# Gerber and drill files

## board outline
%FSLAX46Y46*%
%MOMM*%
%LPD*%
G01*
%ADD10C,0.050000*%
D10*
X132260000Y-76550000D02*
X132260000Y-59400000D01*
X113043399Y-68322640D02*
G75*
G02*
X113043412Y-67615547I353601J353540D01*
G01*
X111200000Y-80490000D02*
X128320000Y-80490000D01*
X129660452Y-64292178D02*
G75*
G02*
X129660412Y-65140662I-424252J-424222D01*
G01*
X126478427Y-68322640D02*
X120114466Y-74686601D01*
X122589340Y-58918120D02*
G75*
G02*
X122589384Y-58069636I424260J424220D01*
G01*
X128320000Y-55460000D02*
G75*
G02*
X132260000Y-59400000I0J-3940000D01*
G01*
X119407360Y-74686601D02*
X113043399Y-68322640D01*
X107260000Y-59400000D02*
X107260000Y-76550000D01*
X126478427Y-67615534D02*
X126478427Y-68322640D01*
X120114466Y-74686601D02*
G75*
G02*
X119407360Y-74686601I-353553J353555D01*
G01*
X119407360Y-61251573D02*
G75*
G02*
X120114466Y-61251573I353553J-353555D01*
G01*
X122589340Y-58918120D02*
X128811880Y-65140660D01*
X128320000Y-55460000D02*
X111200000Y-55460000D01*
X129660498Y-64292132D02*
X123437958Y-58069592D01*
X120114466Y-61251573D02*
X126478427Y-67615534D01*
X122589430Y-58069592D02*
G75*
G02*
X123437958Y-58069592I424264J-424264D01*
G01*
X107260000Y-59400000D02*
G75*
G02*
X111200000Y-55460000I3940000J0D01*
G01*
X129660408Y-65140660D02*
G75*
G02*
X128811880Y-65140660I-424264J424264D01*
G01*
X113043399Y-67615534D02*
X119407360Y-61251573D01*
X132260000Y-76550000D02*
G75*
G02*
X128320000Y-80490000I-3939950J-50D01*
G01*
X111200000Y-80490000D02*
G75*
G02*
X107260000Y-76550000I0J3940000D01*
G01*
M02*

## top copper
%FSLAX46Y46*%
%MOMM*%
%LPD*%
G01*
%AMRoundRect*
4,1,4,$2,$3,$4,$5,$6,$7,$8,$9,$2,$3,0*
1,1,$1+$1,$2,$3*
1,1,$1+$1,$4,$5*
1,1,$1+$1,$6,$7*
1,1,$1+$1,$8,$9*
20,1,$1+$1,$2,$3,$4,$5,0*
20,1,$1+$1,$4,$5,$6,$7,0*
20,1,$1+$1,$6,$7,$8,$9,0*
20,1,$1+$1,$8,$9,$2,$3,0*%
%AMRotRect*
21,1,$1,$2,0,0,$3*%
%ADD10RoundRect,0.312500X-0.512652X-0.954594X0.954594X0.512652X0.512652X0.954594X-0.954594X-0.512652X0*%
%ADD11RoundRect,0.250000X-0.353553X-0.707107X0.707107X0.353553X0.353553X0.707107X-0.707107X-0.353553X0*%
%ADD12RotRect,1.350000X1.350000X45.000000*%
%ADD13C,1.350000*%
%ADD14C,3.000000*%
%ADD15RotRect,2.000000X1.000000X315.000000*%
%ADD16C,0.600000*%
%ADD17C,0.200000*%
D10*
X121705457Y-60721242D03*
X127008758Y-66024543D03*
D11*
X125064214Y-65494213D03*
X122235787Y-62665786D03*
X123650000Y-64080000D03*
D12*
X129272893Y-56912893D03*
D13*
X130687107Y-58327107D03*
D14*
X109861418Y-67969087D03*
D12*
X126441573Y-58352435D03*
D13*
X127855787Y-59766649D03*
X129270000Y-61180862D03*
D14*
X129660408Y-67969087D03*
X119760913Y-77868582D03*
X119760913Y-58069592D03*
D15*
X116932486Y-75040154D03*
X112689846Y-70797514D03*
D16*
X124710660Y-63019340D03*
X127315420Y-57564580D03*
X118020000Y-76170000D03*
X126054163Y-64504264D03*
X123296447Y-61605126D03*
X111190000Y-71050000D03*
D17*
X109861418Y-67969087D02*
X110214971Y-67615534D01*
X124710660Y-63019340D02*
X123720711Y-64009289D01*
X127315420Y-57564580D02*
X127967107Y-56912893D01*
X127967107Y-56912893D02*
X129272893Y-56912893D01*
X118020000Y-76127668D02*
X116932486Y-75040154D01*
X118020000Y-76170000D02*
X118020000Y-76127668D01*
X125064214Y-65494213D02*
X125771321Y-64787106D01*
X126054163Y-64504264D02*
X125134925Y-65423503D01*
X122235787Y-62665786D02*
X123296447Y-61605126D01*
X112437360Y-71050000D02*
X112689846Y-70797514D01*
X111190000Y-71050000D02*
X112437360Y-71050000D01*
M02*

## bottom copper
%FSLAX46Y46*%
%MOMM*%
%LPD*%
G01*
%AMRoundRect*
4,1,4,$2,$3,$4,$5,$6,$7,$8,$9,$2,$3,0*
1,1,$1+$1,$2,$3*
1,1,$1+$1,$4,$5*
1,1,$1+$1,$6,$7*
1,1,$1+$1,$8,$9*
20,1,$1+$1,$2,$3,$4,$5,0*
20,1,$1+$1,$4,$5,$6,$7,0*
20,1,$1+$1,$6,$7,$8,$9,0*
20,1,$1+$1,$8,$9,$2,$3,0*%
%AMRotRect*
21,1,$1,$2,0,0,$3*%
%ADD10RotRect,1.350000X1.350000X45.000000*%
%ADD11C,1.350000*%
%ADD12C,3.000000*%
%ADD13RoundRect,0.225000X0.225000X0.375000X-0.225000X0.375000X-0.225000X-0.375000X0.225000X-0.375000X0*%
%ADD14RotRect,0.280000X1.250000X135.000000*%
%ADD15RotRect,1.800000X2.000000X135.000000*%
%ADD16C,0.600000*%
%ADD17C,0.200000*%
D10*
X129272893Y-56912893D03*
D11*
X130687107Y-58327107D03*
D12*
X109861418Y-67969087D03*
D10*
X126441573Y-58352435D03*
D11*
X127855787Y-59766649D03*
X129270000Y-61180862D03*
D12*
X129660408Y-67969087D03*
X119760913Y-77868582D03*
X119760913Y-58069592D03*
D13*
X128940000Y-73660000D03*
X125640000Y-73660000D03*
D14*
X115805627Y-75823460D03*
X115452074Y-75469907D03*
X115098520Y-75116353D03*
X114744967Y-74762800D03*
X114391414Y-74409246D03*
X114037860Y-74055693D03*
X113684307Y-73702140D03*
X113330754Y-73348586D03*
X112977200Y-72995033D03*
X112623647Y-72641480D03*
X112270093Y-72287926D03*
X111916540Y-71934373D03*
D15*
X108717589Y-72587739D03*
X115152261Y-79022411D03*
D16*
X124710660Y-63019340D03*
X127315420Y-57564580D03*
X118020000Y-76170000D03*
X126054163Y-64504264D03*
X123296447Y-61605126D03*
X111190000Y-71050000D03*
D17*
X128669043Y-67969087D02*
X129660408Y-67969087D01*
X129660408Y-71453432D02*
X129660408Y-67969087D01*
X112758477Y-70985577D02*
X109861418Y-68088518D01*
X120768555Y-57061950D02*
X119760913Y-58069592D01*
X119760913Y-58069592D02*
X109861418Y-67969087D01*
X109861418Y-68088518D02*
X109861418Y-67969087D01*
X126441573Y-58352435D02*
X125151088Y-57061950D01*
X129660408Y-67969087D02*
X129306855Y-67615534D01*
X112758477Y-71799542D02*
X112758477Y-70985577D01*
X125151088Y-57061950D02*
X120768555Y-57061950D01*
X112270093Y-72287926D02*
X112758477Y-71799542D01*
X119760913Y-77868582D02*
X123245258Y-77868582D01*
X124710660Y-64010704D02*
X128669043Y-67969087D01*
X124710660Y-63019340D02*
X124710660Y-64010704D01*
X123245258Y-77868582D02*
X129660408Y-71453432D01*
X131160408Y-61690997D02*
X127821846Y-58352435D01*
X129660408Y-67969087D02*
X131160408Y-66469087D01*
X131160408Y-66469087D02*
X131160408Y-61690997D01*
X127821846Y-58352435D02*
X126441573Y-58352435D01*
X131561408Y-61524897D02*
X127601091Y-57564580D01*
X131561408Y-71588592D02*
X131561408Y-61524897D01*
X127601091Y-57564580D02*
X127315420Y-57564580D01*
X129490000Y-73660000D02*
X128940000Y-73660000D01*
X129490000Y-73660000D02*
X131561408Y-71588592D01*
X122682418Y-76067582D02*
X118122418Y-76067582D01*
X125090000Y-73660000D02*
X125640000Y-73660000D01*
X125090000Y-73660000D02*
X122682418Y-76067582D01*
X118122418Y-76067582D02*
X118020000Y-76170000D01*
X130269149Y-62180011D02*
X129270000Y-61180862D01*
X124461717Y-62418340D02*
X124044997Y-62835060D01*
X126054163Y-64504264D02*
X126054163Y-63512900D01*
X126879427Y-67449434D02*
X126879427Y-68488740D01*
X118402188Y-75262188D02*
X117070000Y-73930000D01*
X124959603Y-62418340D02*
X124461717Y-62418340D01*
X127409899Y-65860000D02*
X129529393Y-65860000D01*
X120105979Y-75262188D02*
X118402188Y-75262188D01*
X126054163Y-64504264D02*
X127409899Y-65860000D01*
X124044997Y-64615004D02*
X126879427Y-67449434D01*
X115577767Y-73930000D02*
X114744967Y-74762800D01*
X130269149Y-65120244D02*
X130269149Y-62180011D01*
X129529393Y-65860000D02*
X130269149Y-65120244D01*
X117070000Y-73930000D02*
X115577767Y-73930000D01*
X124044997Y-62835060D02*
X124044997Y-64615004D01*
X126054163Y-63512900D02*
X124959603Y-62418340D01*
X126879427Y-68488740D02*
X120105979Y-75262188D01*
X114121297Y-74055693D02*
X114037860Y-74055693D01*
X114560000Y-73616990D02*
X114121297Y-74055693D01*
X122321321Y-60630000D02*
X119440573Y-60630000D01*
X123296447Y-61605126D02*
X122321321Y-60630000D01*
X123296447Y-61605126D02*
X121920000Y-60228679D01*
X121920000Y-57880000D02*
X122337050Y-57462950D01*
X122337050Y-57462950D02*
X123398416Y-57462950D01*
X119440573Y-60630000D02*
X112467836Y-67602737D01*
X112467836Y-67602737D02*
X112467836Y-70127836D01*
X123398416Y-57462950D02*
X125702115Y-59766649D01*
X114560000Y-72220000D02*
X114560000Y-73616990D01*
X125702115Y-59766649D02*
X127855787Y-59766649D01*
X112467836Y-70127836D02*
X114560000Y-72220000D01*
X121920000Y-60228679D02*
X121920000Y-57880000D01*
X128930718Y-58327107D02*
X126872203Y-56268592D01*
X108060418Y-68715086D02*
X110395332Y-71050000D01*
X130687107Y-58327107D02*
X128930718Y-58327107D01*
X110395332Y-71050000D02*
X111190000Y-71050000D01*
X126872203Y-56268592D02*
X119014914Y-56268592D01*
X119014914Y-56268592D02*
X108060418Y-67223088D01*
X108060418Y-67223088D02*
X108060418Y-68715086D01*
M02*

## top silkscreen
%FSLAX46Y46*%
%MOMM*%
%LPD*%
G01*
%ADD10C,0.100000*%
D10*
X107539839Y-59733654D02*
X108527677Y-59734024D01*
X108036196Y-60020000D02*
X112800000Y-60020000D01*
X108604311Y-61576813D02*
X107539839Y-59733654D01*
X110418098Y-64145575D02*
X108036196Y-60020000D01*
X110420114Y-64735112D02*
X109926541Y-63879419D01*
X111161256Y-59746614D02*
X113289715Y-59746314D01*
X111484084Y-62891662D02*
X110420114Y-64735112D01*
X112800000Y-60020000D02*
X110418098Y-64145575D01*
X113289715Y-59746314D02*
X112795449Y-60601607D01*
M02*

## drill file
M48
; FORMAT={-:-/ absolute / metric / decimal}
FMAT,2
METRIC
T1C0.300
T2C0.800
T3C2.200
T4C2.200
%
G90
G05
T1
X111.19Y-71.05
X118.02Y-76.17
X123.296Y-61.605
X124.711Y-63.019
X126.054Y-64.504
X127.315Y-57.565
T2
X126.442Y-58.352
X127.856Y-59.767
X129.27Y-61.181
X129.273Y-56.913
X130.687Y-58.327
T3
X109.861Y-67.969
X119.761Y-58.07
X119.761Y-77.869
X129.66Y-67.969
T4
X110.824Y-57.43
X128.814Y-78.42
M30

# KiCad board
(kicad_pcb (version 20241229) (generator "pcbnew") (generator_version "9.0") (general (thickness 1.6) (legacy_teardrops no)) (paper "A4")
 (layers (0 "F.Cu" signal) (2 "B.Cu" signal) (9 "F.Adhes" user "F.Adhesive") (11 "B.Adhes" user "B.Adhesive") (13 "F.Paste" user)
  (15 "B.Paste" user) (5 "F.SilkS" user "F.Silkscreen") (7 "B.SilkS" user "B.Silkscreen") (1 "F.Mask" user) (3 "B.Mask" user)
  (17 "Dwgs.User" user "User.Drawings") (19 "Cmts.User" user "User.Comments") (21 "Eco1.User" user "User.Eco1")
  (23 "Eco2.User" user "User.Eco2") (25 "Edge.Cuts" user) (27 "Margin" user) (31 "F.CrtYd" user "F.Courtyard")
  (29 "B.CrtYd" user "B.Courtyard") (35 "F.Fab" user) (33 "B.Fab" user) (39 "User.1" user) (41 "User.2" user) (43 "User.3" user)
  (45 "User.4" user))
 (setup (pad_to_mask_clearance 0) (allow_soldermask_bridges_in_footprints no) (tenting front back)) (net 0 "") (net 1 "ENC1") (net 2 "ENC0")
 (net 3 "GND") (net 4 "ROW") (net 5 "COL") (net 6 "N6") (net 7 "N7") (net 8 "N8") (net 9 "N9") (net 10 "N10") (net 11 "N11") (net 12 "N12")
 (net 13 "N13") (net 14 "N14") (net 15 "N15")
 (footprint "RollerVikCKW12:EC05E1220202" (layer "F.Cu") (at 119.760913 67.969087 45)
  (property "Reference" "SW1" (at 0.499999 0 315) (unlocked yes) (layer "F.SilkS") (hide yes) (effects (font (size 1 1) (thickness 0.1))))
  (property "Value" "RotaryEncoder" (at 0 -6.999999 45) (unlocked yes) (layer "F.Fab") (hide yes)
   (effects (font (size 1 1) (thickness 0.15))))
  (pad "" smd roundrect (at 6.500001 -3.75 45) (size 2.7 1.25) (layers "F.Cu" "F.Mask" "F.Paste") (roundrect_rratio 0.25)
   (thermal_bridge_angle 45))
  (pad "" smd roundrect (at 6.500001 3.75 45) (size 2.7 1.25) (layers "F.Cu" "F.Mask" "F.Paste") (roundrect_rratio 0.25)
   (thermal_bridge_angle 45))
  (pad "A" smd roundrect (at 5.5 2 45) (size 2 1) (layers "F.Cu" "F.Mask" "F.Paste") (roundrect_rratio 0.25) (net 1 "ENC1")
   (thermal_bridge_angle 45))
  (pad "B" smd roundrect (at 5.5 -2 45) (size 2 1) (layers "F.Cu" "F.Mask" "F.Paste") (roundrect_rratio 0.25) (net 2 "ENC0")
   (thermal_bridge_angle 45))
  (pad "C" smd roundrect (at 5.5 0 45) (size 2 1) (layers "F.Cu" "F.Mask" "F.Paste") (roundrect_rratio 0.25) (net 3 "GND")
   (thermal_bridge_angle 45)))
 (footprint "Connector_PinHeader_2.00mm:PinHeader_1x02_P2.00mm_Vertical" (layer "F.Cu") (at 129.272893 56.912893 45)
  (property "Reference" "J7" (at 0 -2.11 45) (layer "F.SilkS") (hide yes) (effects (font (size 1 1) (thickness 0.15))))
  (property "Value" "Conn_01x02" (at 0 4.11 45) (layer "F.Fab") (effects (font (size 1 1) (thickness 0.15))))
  (pad "1" thru_hole rect (at 0 0 45) (size 1.35 1.35) (drill 0.8) (layers "*.Cu" "*.Mask") (remove_unused_layers no) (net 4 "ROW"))
  (pad "2" thru_hole circle (at 0 2.000001 45) (size 1.35 1.35) (drill 0.8) (layers "*.Cu" "*.Mask") (remove_unused_layers no) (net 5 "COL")))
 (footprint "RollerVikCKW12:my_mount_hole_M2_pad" (layer "F.Cu") (at 109.861418 67.969087 -45)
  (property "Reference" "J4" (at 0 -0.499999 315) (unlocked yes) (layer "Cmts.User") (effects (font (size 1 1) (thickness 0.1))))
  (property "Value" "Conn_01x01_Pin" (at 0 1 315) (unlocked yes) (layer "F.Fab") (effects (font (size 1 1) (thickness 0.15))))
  (pad "1" thru_hole circle (at 0 0 315) (size 3 3) (drill 2.2) (layers "*.Cu" "*.Mask") (remove_unused_layers no) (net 3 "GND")))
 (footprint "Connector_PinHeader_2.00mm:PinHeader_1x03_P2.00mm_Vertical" (layer "F.Cu") (at 126.441573 58.352435 45)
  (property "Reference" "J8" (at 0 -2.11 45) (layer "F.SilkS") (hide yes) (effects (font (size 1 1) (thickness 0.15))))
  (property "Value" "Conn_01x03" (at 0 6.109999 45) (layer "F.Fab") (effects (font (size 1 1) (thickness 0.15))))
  (pad "1" thru_hole rect (at 0 0 45) (size 1.35 1.35) (drill 0.8) (layers "*.Cu" "*.Mask") (remove_unused_layers no) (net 3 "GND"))
  (pad "2" thru_hole circle (at 0 2.000001 45) (size 1.35 1.35) (drill 0.8) (layers "*.Cu" "*.Mask") (remove_unused_layers no)
   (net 2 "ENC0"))
  (pad "3" thru_hole circle (at 0 4 45) (size 1.35 1.35) (drill 0.8) (layers "*.Cu" "*.Mask") (remove_unused_layers no) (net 1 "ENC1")))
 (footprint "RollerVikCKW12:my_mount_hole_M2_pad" (layer "F.Cu") (at 129.660408 67.969087 45)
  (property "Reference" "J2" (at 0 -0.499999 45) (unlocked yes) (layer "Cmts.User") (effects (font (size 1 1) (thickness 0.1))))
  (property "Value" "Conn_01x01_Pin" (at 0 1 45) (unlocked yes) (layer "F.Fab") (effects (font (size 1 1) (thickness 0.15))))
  (pad "1" thru_hole circle (at 0 0 45) (size 3 3) (drill 2.2) (layers "*.Cu" "*.Mask") (remove_unused_layers no) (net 3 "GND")))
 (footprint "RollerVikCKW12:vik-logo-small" (layer "F.Cu") (at 110.42 61.54)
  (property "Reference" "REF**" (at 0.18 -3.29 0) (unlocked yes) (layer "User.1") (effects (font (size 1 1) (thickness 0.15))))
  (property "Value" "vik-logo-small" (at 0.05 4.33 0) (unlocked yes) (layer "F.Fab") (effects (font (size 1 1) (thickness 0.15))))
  (fp_line (start -2.880161 -1.806346) (end -1.892323 -1.805976) (stroke (width 0.1) (type solid)) (layer "F.SilkS"))
  (fp_line (start -2.383804 -1.52) (end 2.38 -1.52) (stroke (width 0.1) (type solid)) (layer "F.SilkS"))
  (fp_line (start -1.815689 0.036813) (end -2.880161 -1.806346) (stroke (width 0.1) (type solid)) (layer "F.SilkS"))
  (fp_line (start -0.001902 2.605575) (end -2.383804 -1.52) (stroke (width 0.1) (type solid)) (layer "F.SilkS"))
  (fp_line (start 0.000114 3.195112) (end -0.493459 2.339419) (stroke (width 0.1) (type solid)) (layer "F.SilkS"))
  (fp_line (start 0.741256 -1.793386) (end 2.869715 -1.793686) (stroke (width 0.1) (type solid)) (layer "F.SilkS"))
  (fp_line (start 1.064084 1.351662) (end 0.000114 3.195112) (stroke (width 0.1) (type solid)) (layer "F.SilkS"))
  (fp_line (start 2.38 -1.52) (end -0.001902 2.605575) (stroke (width 0.1) (type solid)) (layer "F.SilkS"))
  (fp_line (start 2.869715 -1.793686) (end 2.375449 -0.938393) (stroke (width 0.1) (type solid)) (layer "F.SilkS")))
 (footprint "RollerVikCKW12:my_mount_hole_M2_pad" (layer "F.Cu") (at 119.760913 77.868582 135)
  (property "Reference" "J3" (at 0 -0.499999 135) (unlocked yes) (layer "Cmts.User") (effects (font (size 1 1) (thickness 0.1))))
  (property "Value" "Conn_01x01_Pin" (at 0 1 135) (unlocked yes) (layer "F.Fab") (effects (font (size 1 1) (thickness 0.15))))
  (pad "1" thru_hole circle (at 0 0 135) (size 3 3) (drill 2.2) (layers "*.Cu" "*.Mask") (remove_unused_layers no) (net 3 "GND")))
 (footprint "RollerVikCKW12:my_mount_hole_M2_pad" (layer "F.Cu") (at 119.760913 58.069592 45)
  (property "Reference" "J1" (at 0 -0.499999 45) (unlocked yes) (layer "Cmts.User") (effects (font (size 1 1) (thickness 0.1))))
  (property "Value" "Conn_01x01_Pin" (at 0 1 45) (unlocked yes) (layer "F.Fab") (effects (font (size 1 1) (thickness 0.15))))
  (pad "1" thru_hole circle (at 0 0 45) (size 3 3) (drill 2.2) (layers "*.Cu" "*.Mask") (remove_unused_layers no) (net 3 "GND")))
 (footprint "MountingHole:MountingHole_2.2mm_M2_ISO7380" (layer "F.Cu") (at 110.823806 57.429728)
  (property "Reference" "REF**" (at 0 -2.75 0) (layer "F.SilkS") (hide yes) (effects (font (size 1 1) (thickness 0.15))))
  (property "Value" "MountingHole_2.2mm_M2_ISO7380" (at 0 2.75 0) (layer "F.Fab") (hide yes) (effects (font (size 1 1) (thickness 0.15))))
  (pad "" np_thru_hole circle (at 0 0) (size 2.2 2.2) (drill 2.2) (layers "*.Cu" "*.Mask")))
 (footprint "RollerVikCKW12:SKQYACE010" (layer "F.Cu") (at 114.811166 72.918834 -45)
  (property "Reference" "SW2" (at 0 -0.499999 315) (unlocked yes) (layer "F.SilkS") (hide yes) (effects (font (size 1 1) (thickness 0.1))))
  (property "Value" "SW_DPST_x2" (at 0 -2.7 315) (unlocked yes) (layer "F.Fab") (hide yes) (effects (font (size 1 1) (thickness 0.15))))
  (pad "1" smd rect (at 3 0 315) (size 2 1) (layers "F.Cu" "F.Mask" "F.Paste") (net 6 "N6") (thermal_bridge_angle 45))
  (pad "2" smd rect (at -3 0 315) (size 2 1) (layers "F.Cu" "F.Mask" "F.Paste") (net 5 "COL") (thermal_bridge_angle 45)))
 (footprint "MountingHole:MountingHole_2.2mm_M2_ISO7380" (layer "F.Cu") (at 128.813806 78.419728 90)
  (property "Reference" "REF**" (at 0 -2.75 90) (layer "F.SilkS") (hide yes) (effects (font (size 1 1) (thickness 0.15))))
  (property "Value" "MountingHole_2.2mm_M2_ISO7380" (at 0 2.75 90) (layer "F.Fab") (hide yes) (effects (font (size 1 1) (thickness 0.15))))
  (pad "" np_thru_hole circle (at 0 0 90) (size 2.2 2.2) (drill 2.2) (layers "*.Cu" "*.Mask")))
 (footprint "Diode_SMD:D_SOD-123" (layer "B.Cu") (at 127.29 73.66 180)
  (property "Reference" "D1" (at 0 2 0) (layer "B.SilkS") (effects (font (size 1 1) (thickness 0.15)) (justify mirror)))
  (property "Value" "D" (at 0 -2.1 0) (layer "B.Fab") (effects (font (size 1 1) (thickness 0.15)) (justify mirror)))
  (pad "1" smd roundrect (at -1.65 0 180) (size 0.9 1.2) (layers "B.Cu" "B.Mask" "B.Paste") (roundrect_rratio 0.25) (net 4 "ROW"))
  (pad "2" smd roundrect (at 1.65 0 180) (size 0.9 1.2) (layers "B.Cu" "B.Mask" "B.Paste") (roundrect_rratio 0.25) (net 6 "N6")))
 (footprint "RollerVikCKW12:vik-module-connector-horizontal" (layer "B.Cu") (at 112.42 75.32 135)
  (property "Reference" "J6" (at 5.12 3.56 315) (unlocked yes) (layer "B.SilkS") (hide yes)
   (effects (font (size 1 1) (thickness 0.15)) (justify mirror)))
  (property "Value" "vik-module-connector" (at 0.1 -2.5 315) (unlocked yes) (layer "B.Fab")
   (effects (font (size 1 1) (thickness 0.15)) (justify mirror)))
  (pad "1" smd rect (at -2.75 2.038 135) (size 0.28 1.25) (layers "B.Cu" "B.Mask" "B.Paste") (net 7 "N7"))
  (pad "2" smd rect (at -2.25 2.038 135) (size 0.28 1.25) (layers "B.Cu" "B.Mask" "B.Paste") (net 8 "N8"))
  (pad "3" smd rect (at -1.749999 2.038 135) (size 0.28 1.25) (layers "B.Cu" "B.Mask" "B.Paste") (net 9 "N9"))
  (pad "4" smd rect (at -1.25 2.038 135) (size 0.28 1.25) (layers "B.Cu" "B.Mask" "B.Paste") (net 1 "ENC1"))
  (pad "5" smd rect (at -0.75 2.038001 135) (size 0.28 1.25) (layers "B.Cu" "B.Mask" "B.Paste") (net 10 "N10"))
  (pad "6" smd rect (at -0.25 2.038 135) (size 0.28 1.25) (layers "B.Cu" "B.Mask" "B.Paste") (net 2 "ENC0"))
  (pad "7" smd rect (at 0.25 2.038 135) (size 0.28 1.25) (layers "B.Cu" "B.Mask" "B.Paste") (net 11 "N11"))
  (pad "8" smd rect (at 0.75 2.038001 135) (size 0.28 1.25) (layers "B.Cu" "B.Mask" "B.Paste") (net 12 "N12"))
  (pad "9" smd rect (at 1.25 2.038 135) (size 0.28 1.25) (layers "B.Cu" "B.Mask" "B.Paste") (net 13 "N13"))
  (pad "10" smd rect (at 1.749999 2.038 135) (size 0.28 1.25) (layers "B.Cu" "B.Mask" "B.Paste") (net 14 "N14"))
  (pad "11" smd rect (at 2.25 2.038 135) (size 0.28 1.25) (layers "B.Cu" "B.Mask" "B.Paste") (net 3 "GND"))
  (pad "12" smd rect (at 2.75 2.038 135) (size 0.28 1.25) (layers "B.Cu" "B.Mask" "B.Paste") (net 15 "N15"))
  (pad "13" smd rect (at 4.55 -0.686 135) (size 1.8 2) (layers "B.Cu" "B.Mask" "B.Paste"))
  (pad "14" smd rect (at -4.55 -0.686 135) (size 1.8 2) (layers "B.Cu" "B.Mask" "B.Paste")))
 (gr_line (start 132.26 76.55) (end 132.26 59.4) (stroke (width 0.05) (type solid)) (layer "Edge.Cuts"))
 (gr_arc (start 113.043399 68.32264) (mid 112.896953 67.969087) (end 113.043399 67.615534) (stroke (width 0.05) (type default))
  (layer "Edge.Cuts"))
 (gr_line (start 111.2 80.49) (end 128.32 80.49) (stroke (width 0.05) (type solid)) (layer "Edge.Cuts"))
 (gr_arc (start 129.660452 64.292178) (mid 129.836169 64.716427) (end 129.660408 65.140658) (stroke (width 0.05) (type default))
  (layer "Edge.Cuts"))
 (gr_line (start 126.478427 68.32264) (end 120.114466 74.686601) (stroke (width 0.05) (type default)) (layer "Edge.Cuts"))
 (gr_arc (start 122.58934 58.91812) (mid 122.413604 58.493856) (end 122.58934 58.069592) (stroke (width 0.05) (type default))
  (layer "Edge.Cuts"))
 (gr_arc (start 128.32 55.46) (mid 131.10601 56.61399) (end 132.26 59.4) (stroke (width 0.05) (type solid)) (layer "Edge.Cuts"))
 (gr_line (start 119.40736 74.686601) (end 113.043399 68.32264) (stroke (width 0.05) (type default)) (layer "Edge.Cuts"))
 (gr_line (start 107.26 59.4) (end 107.26 76.55) (stroke (width 0.05) (type solid)) (layer "Edge.Cuts"))
 (gr_line (start 126.478427 67.615534) (end 126.478427 68.32264) (stroke (width 0.05) (type default)) (layer "Edge.Cuts"))
 (gr_arc (start 120.114466 74.686601) (mid 119.760913 74.833047) (end 119.40736 74.686601) (stroke (width 0.05) (type default))
  (layer "Edge.Cuts"))
 (gr_arc (start 119.40736 61.251573) (mid 119.760913 61.105127) (end 120.114466 61.251573) (stroke (width 0.05) (type default))
  (layer "Edge.Cuts"))
 (gr_line (start 122.58934 58.91812) (end 128.81188 65.14066) (stroke (width 0.05) (type default)) (layer "Edge.Cuts"))
 (gr_line (start 128.32 55.46) (end 111.2 55.46) (stroke (width 0.05) (type solid)) (layer "Edge.Cuts"))
 (gr_line (start 129.660498 64.292132) (end 123.437958 58.069592) (stroke (width 0.05) (type default)) (layer "Edge.Cuts"))
 (gr_line (start 120.114466 61.251573) (end 126.478427 67.615534) (stroke (width 0.05) (type default)) (layer "Edge.Cuts"))
 (gr_arc (start 122.58943 58.069592) (mid 123.013694 57.893856) (end 123.437958 58.069592) (stroke (width 0.05) (type default))
  (layer "Edge.Cuts"))
 (gr_arc (start 107.26 59.4) (mid 108.414 56.614) (end 111.2 55.46) (stroke (width 0.05) (type solid)) (layer "Edge.Cuts"))
 (gr_arc (start 129.660408 65.14066) (mid 129.236144 65.316396) (end 128.81188 65.14066) (stroke (width 0.05) (type default))
  (layer "Edge.Cuts"))
 (gr_line (start 113.043399 67.615534) (end 119.40736 61.251573) (stroke (width 0.05) (type default)) (layer "Edge.Cuts"))
 (gr_arc (start 132.26 76.55) (mid 131.106014 79.336014) (end 128.32 80.49) (stroke (width 0.05) (type solid)) (layer "Edge.Cuts"))
 (gr_arc (start 111.2 80.49) (mid 108.414008 79.335992) (end 107.26 76.55) (stroke (width 0.05) (type solid)) (layer "Edge.Cuts"))
 (segment (start 109.861418 67.969087) (end 110.214971 67.615534) (width 0.2) (layer "F.Cu") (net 3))
 (segment (start 124.71066 63.01934) (end 123.720711 64.009289) (width 0.2) (layer "F.Cu") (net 3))
 (via (at 124.71066 63.01934) (size 0.6) (drill 0.3) (layers "F.Cu" "B.Cu") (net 3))
 (segment (start 128.669043 67.969087) (end 129.660408 67.969087) (width 0.2) (layer "B.Cu") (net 3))
 (segment (start 129.660408 71.453432) (end 129.660408 67.969087) (width 0.2) (layer "B.Cu") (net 3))
 (segment (start 112.758477 70.985577) (end 109.861418 68.088518) (width 0.2) (layer "B.Cu") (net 3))
 (segment (start 120.768555 57.06195) (end 119.760913 58.069592) (width 0.2) (layer "B.Cu") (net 3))
 (segment (start 119.760913 58.069592) (end 109.861418 67.969087) (width 0.2) (layer "B.Cu") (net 3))
 (segment (start 109.861418 68.088518) (end 109.861418 67.969087) (width 0.2) (layer "B.Cu") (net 3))
 (segment (start 126.441573 58.352435) (end 125.151088 57.06195) (width 0.2) (layer "B.Cu") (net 3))
 (segment (start 129.660408 67.969087) (end 129.306855 67.615534) (width 0.2) (layer "B.Cu") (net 3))
 (segment (start 112.758477 71.799542) (end 112.758477 70.985577) (width 0.2) (layer "B.Cu") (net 3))
 (segment (start 125.151088 57.06195) (end 120.768555 57.06195) (width 0.2) (layer "B.Cu") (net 3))
 (segment (start 112.270093 72.287926) (end 112.758477 71.799542) (width 0.2) (layer "B.Cu") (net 3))
 (segment (start 119.760913 77.868582) (end 123.245258 77.868582) (width 0.2) (layer "B.Cu") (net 3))
 (segment (start 124.71066 64.010704) (end 128.669043 67.969087) (width 0.2) (layer "B.Cu") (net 3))
 (segment (start 124.71066 63.01934) (end 124.71066 64.010704) (width 0.2) (layer "B.Cu") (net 3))
 (segment (start 123.245258 77.868582) (end 129.660408 71.453432) (width 0.2) (layer "B.Cu") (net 3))
 (segment (start 131.160408 61.690997) (end 127.821846 58.352435) (width 0.2) (layer "B.Cu") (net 3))
 (segment (start 129.660408 67.969087) (end 131.160408 66.469087) (width 0.2) (layer "B.Cu") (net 3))
 (segment (start 131.160408 66.469087) (end 131.160408 61.690997) (width 0.2) (layer "B.Cu") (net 3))
 (segment (start 127.821846 58.352435) (end 126.441573 58.352435) (width 0.2) (layer "B.Cu") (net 3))
 (segment (start 127.31542 57.56458) (end 127.967107 56.912893) (width 0.2) (layer "F.Cu") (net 4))
 (segment (start 127.967107 56.912893) (end 129.272893 56.912893) (width 0.2) (layer "F.Cu") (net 4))
 (via (at 127.31542 57.56458) (size 0.6) (drill 0.3) (layers "F.Cu" "B.Cu") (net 4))
 (segment (start 131.561408 61.524897) (end 127.601091 57.56458) (width 0.2) (layer "B.Cu") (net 4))
 (segment (start 131.561408 71.588592) (end 131.561408 61.524897) (width 0.2) (layer "B.Cu") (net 4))
 (segment (start 127.601091 57.56458) (end 127.31542 57.56458) (width 0.2) (layer "B.Cu") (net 4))
 (segment (start 129.49 73.66) (end 128.94 73.66) (width 0.2) (layer "B.Cu") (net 4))
 (segment (start 129.49 73.66) (end 131.561408 71.588592) (width 0.2) (layer "B.Cu") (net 4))
 (segment (start 118.02 76.127668) (end 116.932486 75.040154) (width 0.2) (layer "F.Cu") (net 6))
 (segment (start 118.02 76.17) (end 118.02 76.127668) (width 0.2) (layer "F.Cu") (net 6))
 (via (at 118.02 76.17) (size 0.6) (drill 0.3) (layers "F.Cu" "B.Cu") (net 6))
 (segment (start 122.682418 76.067582) (end 118.122418 76.067582) (width 0.2) (layer "B.Cu") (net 6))
 (segment (start 125.09 73.66) (end 125.64 73.66) (width 0.2) (layer "B.Cu") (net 6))
 (segment (start 125.09 73.66) (end 122.682418 76.067582) (width 0.2) (layer "B.Cu") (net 6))
 (segment (start 118.122418 76.067582) (end 118.02 76.17) (width 0.2) (layer "B.Cu") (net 6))
 (segment (start 125.064214 65.494213) (end 125.771321 64.787106) (width 0.2) (layer "F.Cu") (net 1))
 (segment (start 126.054163 64.504264) (end 125.134925 65.423503) (width 0.2) (layer "F.Cu") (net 1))
 (via (at 126.054163 64.504264) (size 0.6) (drill 0.3) (layers "F.Cu" "B.Cu") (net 1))
 (segment (start 130.269149 62.180011) (end 129.27 61.180862) (width 0.2) (layer "B.Cu") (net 1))
 (segment (start 124.461717 62.41834) (end 124.044997 62.83506) (width 0.2) (layer "B.Cu") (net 1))
 (segment (start 126.054163 64.504264) (end 126.054163 63.5129) (width 0.2) (layer "B.Cu") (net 1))
 (segment (start 126.879427 67.449434) (end 126.879427 68.48874) (width 0.2) (layer "B.Cu") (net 1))
 (segment (start 118.402188 75.262188) (end 117.07 73.93) (width 0.2) (layer "B.Cu") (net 1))
 (segment (start 124.959603 62.41834) (end 124.461717 62.41834) (width 0.2) (layer "B.Cu") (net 1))
 (segment (start 127.409899 65.86) (end 129.529393 65.86) (width 0.2) (layer "B.Cu") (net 1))
 (segment (start 120.105979 75.262188) (end 118.402188 75.262188) (width 0.2) (layer "B.Cu") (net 1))
 (segment (start 126.054163 64.504264) (end 127.409899 65.86) (width 0.2) (layer "B.Cu") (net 1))
 (segment (start 124.044997 64.615004) (end 126.879427 67.449434) (width 0.2) (layer "B.Cu") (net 1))
 (segment (start 115.577767 73.93) (end 114.744967 74.7628) (width 0.2) (layer "B.Cu") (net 1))
 (segment (start 130.269149 65.120244) (end 130.269149 62.180011) (width 0.2) (layer "B.Cu") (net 1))
 (segment (start 129.529393 65.86) (end 130.269149 65.120244) (width 0.2) (layer "B.Cu") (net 1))
 (segment (start 117.07 73.93) (end 115.577767 73.93) (width 0.2) (layer "B.Cu") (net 1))
 (segment (start 124.044997 62.83506) (end 124.044997 64.615004) (width 0.2) (layer "B.Cu") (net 1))
 (segment (start 126.054163 63.5129) (end 124.959603 62.41834) (width 0.2) (layer "B.Cu") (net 1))
 (segment (start 126.879427 68.48874) (end 120.105979 75.262188) (width 0.2) (layer "B.Cu") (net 1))
 (segment (start 122.235787 62.665786) (end 123.296447 61.605126) (width 0.2) (layer "F.Cu") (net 2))
 (via (at 123.296447 61.605126) (size 0.6) (drill 0.3) (layers "F.Cu" "B.Cu") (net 2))
 (segment (start 114.121297 74.055693) (end 114.03786 74.055693) (width 0.2) (layer "B.Cu") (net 2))
 (segment (start 114.56 73.61699) (end 114.121297 74.055693) (width 0.2) (layer "B.Cu") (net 2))
 (segment (start 122.321321 60.63) (end 119.440573 60.63) (width 0.2) (layer "B.Cu") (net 2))
 (segment (start 123.296447 61.605126) (end 122.321321 60.63) (width 0.2) (layer "B.Cu") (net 2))
 (segment (start 123.296447 61.605126) (end 121.92 60.228679) (width 0.2) (layer "B.Cu") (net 2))
 (segment (start 121.92 57.88) (end 122.33705 57.46295) (width 0.2) (layer "B.Cu") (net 2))
 (segment (start 122.33705 57.46295) (end 123.398416 57.46295) (width 0.2) (layer "B.Cu") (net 2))
 (segment (start 119.440573 60.63) (end 112.467836 67.602737) (width 0.2) (layer "B.Cu") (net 2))
 (segment (start 112.467836 67.602737) (end 112.467836 70.127836) (width 0.2) (layer "B.Cu") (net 2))
 (segment (start 123.398416 57.46295) (end 125.702115 59.766649) (width 0.2) (layer "B.Cu") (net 2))
 (segment (start 114.56 72.22) (end 114.56 73.61699) (width 0.2) (layer "B.Cu") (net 2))
 (segment (start 125.702115 59.766649) (end 127.855787 59.766649) (width 0.2) (layer "B.Cu") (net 2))
 (segment (start 112.467836 70.127836) (end 114.56 72.22) (width 0.2) (layer "B.Cu") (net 2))
 (segment (start 121.92 60.228679) (end 121.92 57.88) (width 0.2) (layer "B.Cu") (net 2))
 (segment (start 112.43736 71.05) (end 112.689846 70.797514) (width 0.2) (layer "F.Cu") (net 5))
 (segment (start 111.19 71.05) (end 112.43736 71.05) (width 0.2) (layer "F.Cu") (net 5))
 (via (at 111.19 71.05) (size 0.6) (drill 0.3) (layers "F.Cu" "B.Cu") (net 5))
 (segment (start 128.930718 58.327107) (end 126.872203 56.268592) (width 0.2) (layer "B.Cu") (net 5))
 (segment (start 108.060418 68.715086) (end 110.395332 71.05) (width 0.2) (layer "B.Cu") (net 5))
 (segment (start 130.687107 58.327107) (end 128.930718 58.327107) (width 0.2) (layer "B.Cu") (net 5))
 (segment (start 110.395332 71.05) (end 111.19 71.05) (width 0.2) (layer "B.Cu") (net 5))
 (segment (start 126.872203 56.268592) (end 119.014914 56.268592) (width 0.2) (layer "B.Cu") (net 5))
 (segment (start 119.014914 56.268592) (end 108.060418 67.223088) (width 0.2) (layer "B.Cu") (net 5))
 (segment (start 108.060418 67.223088) (end 108.060418 68.715086) (width 0.2) (layer "B.Cu") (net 5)))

